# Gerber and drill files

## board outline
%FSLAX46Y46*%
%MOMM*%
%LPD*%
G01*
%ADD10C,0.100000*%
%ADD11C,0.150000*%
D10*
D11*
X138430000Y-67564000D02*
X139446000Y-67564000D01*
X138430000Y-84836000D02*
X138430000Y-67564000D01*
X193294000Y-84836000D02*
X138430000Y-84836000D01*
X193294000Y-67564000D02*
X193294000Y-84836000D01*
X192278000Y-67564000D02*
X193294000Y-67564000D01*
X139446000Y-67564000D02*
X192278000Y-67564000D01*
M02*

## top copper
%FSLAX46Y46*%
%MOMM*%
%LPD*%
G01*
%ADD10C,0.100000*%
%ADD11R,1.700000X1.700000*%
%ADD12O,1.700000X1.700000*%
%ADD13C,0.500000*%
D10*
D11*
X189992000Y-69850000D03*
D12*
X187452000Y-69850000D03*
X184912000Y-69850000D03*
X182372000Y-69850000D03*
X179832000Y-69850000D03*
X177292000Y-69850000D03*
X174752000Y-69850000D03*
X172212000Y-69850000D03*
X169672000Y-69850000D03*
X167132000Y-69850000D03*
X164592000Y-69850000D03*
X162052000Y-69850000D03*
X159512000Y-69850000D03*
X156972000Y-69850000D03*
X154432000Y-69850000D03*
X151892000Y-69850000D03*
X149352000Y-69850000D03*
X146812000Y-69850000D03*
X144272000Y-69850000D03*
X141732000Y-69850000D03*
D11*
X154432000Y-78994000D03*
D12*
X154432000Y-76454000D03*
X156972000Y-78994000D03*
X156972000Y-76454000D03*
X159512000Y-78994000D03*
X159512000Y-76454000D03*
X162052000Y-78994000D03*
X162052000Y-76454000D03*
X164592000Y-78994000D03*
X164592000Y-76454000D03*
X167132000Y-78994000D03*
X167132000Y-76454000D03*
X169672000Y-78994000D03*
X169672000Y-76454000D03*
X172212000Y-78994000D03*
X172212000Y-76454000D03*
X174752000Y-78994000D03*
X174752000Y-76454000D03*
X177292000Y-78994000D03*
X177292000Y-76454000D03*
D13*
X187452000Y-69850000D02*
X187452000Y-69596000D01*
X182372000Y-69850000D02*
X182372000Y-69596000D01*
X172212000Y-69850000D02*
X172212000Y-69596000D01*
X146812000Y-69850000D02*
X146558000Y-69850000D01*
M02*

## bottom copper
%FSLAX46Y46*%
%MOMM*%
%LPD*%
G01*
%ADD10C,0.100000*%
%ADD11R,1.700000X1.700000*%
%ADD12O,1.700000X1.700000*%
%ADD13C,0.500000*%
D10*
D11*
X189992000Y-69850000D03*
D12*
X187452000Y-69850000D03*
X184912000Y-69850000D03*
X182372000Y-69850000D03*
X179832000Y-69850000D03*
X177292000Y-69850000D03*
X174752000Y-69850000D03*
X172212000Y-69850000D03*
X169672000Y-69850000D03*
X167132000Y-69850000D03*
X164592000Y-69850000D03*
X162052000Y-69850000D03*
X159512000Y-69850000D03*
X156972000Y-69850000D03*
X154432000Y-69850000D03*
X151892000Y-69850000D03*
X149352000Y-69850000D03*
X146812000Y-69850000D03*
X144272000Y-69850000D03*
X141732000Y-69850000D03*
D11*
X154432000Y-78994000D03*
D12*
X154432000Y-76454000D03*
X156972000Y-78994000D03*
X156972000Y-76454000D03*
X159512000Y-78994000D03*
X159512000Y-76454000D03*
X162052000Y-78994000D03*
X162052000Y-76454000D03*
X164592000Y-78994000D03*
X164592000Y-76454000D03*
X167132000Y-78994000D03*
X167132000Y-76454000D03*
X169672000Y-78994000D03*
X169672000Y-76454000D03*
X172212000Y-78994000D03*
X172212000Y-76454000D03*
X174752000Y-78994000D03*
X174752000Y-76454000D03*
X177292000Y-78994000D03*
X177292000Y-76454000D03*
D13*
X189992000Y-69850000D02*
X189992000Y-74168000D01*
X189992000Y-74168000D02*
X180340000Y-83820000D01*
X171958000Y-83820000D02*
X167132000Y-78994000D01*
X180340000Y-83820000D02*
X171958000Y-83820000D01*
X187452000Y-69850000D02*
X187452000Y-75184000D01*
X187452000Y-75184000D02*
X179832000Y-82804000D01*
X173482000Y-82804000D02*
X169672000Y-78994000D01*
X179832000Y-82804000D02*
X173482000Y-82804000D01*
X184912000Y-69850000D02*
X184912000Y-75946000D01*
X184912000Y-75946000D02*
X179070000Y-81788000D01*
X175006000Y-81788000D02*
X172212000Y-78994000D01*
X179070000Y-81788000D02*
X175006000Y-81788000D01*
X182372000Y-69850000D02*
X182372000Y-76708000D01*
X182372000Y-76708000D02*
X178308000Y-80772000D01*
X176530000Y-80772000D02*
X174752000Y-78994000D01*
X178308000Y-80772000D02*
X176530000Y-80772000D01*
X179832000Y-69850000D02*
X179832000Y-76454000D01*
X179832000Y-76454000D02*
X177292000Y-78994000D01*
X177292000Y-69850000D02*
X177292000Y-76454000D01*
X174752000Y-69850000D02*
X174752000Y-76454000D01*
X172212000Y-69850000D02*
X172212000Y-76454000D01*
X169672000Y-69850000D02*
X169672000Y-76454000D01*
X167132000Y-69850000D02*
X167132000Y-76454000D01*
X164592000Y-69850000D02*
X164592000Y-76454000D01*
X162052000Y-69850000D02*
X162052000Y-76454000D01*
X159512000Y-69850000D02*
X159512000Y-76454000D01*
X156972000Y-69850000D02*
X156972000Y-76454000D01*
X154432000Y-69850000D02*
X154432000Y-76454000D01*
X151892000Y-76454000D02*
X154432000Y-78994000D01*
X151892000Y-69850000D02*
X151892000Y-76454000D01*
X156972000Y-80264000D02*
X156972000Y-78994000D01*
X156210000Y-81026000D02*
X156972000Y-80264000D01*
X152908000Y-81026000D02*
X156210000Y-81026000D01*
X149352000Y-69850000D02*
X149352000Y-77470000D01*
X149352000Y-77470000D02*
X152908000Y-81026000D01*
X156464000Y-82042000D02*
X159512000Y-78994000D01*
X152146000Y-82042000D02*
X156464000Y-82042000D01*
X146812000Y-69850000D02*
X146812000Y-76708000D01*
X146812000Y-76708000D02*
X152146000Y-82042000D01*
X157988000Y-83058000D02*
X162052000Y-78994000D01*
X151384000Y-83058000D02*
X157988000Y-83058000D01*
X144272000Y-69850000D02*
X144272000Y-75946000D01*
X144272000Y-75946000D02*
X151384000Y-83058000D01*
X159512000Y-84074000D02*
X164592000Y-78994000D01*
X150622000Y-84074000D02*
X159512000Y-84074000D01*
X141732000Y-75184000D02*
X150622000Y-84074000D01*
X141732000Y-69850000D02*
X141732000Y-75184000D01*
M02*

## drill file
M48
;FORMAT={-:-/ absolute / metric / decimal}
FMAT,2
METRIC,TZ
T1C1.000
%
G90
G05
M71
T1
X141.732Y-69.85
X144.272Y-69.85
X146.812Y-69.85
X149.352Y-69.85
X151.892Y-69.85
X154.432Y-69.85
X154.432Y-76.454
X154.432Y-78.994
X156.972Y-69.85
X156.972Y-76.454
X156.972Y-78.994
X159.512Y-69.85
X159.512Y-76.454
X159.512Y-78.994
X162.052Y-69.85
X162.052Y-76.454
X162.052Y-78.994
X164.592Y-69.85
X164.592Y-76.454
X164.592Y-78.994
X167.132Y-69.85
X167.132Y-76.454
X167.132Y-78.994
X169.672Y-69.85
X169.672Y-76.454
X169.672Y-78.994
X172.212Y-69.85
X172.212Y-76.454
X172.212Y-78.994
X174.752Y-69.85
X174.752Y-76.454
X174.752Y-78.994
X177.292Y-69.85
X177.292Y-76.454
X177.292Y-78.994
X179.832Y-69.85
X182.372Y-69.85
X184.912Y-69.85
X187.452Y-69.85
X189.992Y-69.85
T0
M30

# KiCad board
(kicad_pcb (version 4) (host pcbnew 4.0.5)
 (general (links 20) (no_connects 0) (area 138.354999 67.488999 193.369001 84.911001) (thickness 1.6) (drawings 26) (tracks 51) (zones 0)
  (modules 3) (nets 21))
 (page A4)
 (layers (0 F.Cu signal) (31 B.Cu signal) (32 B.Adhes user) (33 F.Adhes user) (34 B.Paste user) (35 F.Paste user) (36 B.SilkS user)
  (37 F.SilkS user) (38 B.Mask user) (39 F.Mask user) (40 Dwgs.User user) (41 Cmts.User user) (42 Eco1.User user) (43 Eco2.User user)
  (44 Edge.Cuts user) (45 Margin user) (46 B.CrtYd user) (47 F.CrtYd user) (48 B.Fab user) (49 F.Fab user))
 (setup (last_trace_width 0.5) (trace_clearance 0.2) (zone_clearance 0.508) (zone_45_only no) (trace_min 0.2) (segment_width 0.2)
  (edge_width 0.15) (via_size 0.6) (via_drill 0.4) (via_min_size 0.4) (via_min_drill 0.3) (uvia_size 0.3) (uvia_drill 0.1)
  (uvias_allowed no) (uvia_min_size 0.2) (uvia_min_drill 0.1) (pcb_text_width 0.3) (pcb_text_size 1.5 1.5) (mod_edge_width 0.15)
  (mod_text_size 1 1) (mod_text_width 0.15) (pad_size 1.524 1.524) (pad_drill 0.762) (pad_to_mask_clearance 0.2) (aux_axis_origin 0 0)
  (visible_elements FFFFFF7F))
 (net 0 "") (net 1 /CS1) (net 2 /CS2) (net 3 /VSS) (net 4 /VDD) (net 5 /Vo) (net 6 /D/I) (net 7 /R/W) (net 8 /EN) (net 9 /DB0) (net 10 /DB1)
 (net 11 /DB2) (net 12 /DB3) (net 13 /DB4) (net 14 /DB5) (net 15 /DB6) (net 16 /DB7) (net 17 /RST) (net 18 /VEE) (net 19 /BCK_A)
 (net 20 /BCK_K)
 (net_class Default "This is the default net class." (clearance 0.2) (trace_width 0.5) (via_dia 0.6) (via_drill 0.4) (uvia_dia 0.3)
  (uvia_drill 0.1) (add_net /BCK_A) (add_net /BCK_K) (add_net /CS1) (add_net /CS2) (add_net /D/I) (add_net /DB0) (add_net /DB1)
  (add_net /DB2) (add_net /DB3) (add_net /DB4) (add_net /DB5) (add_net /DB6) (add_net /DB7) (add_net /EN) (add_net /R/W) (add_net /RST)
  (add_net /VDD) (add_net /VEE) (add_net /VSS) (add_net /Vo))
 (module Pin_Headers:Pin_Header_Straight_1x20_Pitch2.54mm (layer F.Cu) (at 189.992 69.85 270)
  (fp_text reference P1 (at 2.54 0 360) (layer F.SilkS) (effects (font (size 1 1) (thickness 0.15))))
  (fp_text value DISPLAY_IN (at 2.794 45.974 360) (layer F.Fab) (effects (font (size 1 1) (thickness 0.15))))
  (pad 1 thru_hole rect (at 0 0 270) (size 1.7 1.7) (drill 1) (layers *.Cu *.Mask) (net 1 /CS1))
  (pad 2 thru_hole oval (at 0 2.54 270) (size 1.7 1.7) (drill 1) (layers *.Cu *.Mask) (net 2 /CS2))
  (pad 3 thru_hole oval (at 0 5.08 270) (size 1.7 1.7) (drill 1) (layers *.Cu *.Mask) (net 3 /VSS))
  (pad 4 thru_hole oval (at 0 7.62 270) (size 1.7 1.7) (drill 1) (layers *.Cu *.Mask) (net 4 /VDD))
  (pad 5 thru_hole oval (at 0 10.16 270) (size 1.7 1.7) (drill 1) (layers *.Cu *.Mask) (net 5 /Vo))
  (pad 6 thru_hole oval (at 0 12.7 270) (size 1.7 1.7) (drill 1) (layers *.Cu *.Mask) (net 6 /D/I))
  (pad 7 thru_hole oval (at 0 15.24 270) (size 1.7 1.7) (drill 1) (layers *.Cu *.Mask) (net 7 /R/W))
  (pad 8 thru_hole oval (at 0 17.78 270) (size 1.7 1.7) (drill 1) (layers *.Cu *.Mask) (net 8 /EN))
  (pad 9 thru_hole oval (at 0 20.32 270) (size 1.7 1.7) (drill 1) (layers *.Cu *.Mask) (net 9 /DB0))
  (pad 10 thru_hole oval (at 0 22.86 270) (size 1.7 1.7) (drill 1) (layers *.Cu *.Mask) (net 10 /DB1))
  (pad 11 thru_hole oval (at 0 25.4 270) (size 1.7 1.7) (drill 1) (layers *.Cu *.Mask) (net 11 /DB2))
  (pad 12 thru_hole oval (at 0 27.94 270) (size 1.7 1.7) (drill 1) (layers *.Cu *.Mask) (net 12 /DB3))
  (pad 13 thru_hole oval (at 0 30.48 270) (size 1.7 1.7) (drill 1) (layers *.Cu *.Mask) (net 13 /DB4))
  (pad 14 thru_hole oval (at 0 33.02 270) (size 1.7 1.7) (drill 1) (layers *.Cu *.Mask) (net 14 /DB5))
  (pad 15 thru_hole oval (at 0 35.56 270) (size 1.7 1.7) (drill 1) (layers *.Cu *.Mask) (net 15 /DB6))
  (pad 16 thru_hole oval (at 0 38.1 270) (size 1.7 1.7) (drill 1) (layers *.Cu *.Mask) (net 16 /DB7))
  (pad 17 thru_hole oval (at 0 40.64 270) (size 1.7 1.7) (drill 1) (layers *.Cu *.Mask) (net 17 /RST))
  (pad 18 thru_hole oval (at 0 43.18 270) (size 1.7 1.7) (drill 1) (layers *.Cu *.Mask) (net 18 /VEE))
  (pad 19 thru_hole oval (at 0 45.72 270) (size 1.7 1.7) (drill 1) (layers *.Cu *.Mask) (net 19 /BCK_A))
  (pad 20 thru_hole oval (at 0 48.26 270) (size 1.7 1.7) (drill 1) (layers *.Cu *.Mask) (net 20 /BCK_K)))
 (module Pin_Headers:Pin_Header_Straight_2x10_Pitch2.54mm (layer F.Cu) (at 154.432 78.994 90)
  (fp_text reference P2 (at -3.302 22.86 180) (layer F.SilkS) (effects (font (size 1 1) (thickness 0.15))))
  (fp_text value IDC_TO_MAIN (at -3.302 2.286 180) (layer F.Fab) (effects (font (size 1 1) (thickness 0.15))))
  (pad 1 thru_hole rect (at 0 0 90) (size 1.7 1.7) (drill 1) (layers *.Cu *.Mask) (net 16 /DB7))
  (pad 2 thru_hole oval (at 2.54 0 90) (size 1.7 1.7) (drill 1) (layers *.Cu *.Mask) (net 15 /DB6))
  (pad 3 thru_hole oval (at 0 2.54 90) (size 1.7 1.7) (drill 1) (layers *.Cu *.Mask) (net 17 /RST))
  (pad 4 thru_hole oval (at 2.54 2.54 90) (size 1.7 1.7) (drill 1) (layers *.Cu *.Mask) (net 14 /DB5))
  (pad 5 thru_hole oval (at 0 5.08 90) (size 1.7 1.7) (drill 1) (layers *.Cu *.Mask) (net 18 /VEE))
  (pad 6 thru_hole oval (at 2.54 5.08 90) (size 1.7 1.7) (drill 1) (layers *.Cu *.Mask) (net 13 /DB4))
  (pad 7 thru_hole oval (at 0 7.62 90) (size 1.7 1.7) (drill 1) (layers *.Cu *.Mask) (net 19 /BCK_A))
  (pad 8 thru_hole oval (at 2.54 7.62 90) (size 1.7 1.7) (drill 1) (layers *.Cu *.Mask) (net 12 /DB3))
  (pad 9 thru_hole oval (at 0 10.16 90) (size 1.7 1.7) (drill 1) (layers *.Cu *.Mask) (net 20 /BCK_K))
  (pad 10 thru_hole oval (at 2.54 10.16 90) (size 1.7 1.7) (drill 1) (layers *.Cu *.Mask) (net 11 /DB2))
  (pad 11 thru_hole oval (at 0 12.7 90) (size 1.7 1.7) (drill 1) (layers *.Cu *.Mask) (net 1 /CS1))
  (pad 12 thru_hole oval (at 2.54 12.7 90) (size 1.7 1.7) (drill 1) (layers *.Cu *.Mask) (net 10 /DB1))
  (pad 13 thru_hole oval (at 0 15.24 90) (size 1.7 1.7) (drill 1) (layers *.Cu *.Mask) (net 2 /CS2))
  (pad 14 thru_hole oval (at 2.54 15.24 90) (size 1.7 1.7) (drill 1) (layers *.Cu *.Mask) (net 9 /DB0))
  (pad 15 thru_hole oval (at 0 17.78 90) (size 1.7 1.7) (drill 1) (layers *.Cu *.Mask) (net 3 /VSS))
  (pad 16 thru_hole oval (at 2.54 17.78 90) (size 1.7 1.7) (drill 1) (layers *.Cu *.Mask) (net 8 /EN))
  (pad 17 thru_hole oval (at 0 20.32 90) (size 1.7 1.7) (drill 1) (layers *.Cu *.Mask) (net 4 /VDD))
  (pad 18 thru_hole oval (at 2.54 20.32 90) (size 1.7 1.7) (drill 1) (layers *.Cu *.Mask) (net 7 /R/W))
  (pad 19 thru_hole oval (at 0 22.86 90) (size 1.7 1.7) (drill 1) (layers *.Cu *.Mask) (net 5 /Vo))
  (pad 20 thru_hole oval (at 2.54 22.86 90) (size 1.7 1.7) (drill 1) (layers *.Cu *.Mask) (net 6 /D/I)))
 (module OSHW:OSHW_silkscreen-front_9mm (layer F.Cu) (at 145.288 78.994)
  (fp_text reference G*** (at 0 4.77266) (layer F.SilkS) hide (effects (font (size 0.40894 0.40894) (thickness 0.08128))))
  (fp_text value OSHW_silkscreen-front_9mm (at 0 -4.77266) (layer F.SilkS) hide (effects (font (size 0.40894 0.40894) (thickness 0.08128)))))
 (gr_line (start 138.43 67.564) (end 139.446 67.564) (angle 90) (layer Edge.Cuts) (width 0.15))
 (gr_line (start 138.43 84.836) (end 138.43 67.564) (angle 90) (layer Edge.Cuts) (width 0.15))
 (gr_line (start 193.294 84.836) (end 138.43 84.836) (angle 90) (layer Edge.Cuts) (width 0.15))
 (gr_line (start 193.294 67.564) (end 193.294 84.836) (angle 90) (layer Edge.Cuts) (width 0.15))
 (gr_line (start 192.278 67.564) (end 193.294 67.564) (angle 90) (layer Edge.Cuts) (width 0.15))
 (gr_line (start 139.446 67.564) (end 192.278 67.564) (angle 90) (layer Edge.Cuts) (width 0.15))
 (segment (start 189.992 69.85) (end 189.992 74.168) (width 0.5) (layer B.Cu) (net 1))
 (segment (start 189.992 74.168) (end 180.34 83.82) (width 0.5) (layer B.Cu) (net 1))
 (segment (start 171.958 83.82) (end 167.132 78.994) (width 0.5) (layer B.Cu) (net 1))
 (segment (start 180.34 83.82) (end 171.958 83.82) (width 0.5) (layer B.Cu) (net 1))
 (segment (start 187.452 69.85) (end 187.452 69.596) (width 0.5) (layer F.Cu) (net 2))
 (segment (start 187.452 69.85) (end 187.452 75.184) (width 0.5) (layer B.Cu) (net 2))
 (segment (start 187.452 75.184) (end 179.832 82.804) (width 0.5) (layer B.Cu) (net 2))
 (segment (start 173.482 82.804) (end 169.672 78.994) (width 0.5) (layer B.Cu) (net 2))
 (segment (start 179.832 82.804) (end 173.482 82.804) (width 0.5) (layer B.Cu) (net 2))
 (segment (start 184.912 69.85) (end 184.912 75.946) (width 0.5) (layer B.Cu) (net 3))
 (segment (start 184.912 75.946) (end 179.07 81.788) (width 0.5) (layer B.Cu) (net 3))
 (segment (start 175.006 81.788) (end 172.212 78.994) (width 0.5) (layer B.Cu) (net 3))
 (segment (start 179.07 81.788) (end 175.006 81.788) (width 0.5) (layer B.Cu) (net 3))
 (segment (start 182.372 69.85) (end 182.372 69.596) (width 0.5) (layer F.Cu) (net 4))
 (segment (start 182.372 69.85) (end 182.372 76.708) (width 0.5) (layer B.Cu) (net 4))
 (segment (start 182.372 76.708) (end 178.308 80.772) (width 0.5) (layer B.Cu) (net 4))
 (segment (start 176.53 80.772) (end 174.752 78.994) (width 0.5) (layer B.Cu) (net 4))
 (segment (start 178.308 80.772) (end 176.53 80.772) (width 0.5) (layer B.Cu) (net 4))
 (segment (start 179.832 69.85) (end 179.832 76.454) (width 0.5) (layer B.Cu) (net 5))
 (segment (start 179.832 76.454) (end 177.292 78.994) (width 0.5) (layer B.Cu) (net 5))
 (segment (start 177.292 69.85) (end 177.292 76.454) (width 0.5) (layer B.Cu) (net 6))
 (segment (start 174.752 69.85) (end 174.752 76.454) (width 0.5) (layer B.Cu) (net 7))
 (segment (start 172.212 69.85) (end 172.212 69.596) (width 0.5) (layer F.Cu) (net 8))
 (segment (start 172.212 69.85) (end 172.212 76.454) (width 0.5) (layer B.Cu) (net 8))
 (segment (start 169.672 69.85) (end 169.672 76.454) (width 0.5) (layer B.Cu) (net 9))
 (segment (start 167.132 69.85) (end 167.132 76.454) (width 0.5) (layer B.Cu) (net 10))
 (segment (start 164.592 69.85) (end 164.592 76.454) (width 0.5) (layer B.Cu) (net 11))
 (segment (start 162.052 69.85) (end 162.052 76.454) (width 0.5) (layer B.Cu) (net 12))
 (segment (start 159.512 69.85) (end 159.512 76.454) (width 0.5) (layer B.Cu) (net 13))
 (segment (start 156.972 69.85) (end 156.972 76.454) (width 0.5) (layer B.Cu) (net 14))
 (segment (start 154.432 69.85) (end 154.432 76.454) (width 0.5) (layer B.Cu) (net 15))
 (segment (start 151.892 76.454) (end 154.432 78.994) (width 0.5) (layer B.Cu) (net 16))
 (segment (start 151.892 69.85) (end 151.892 76.454) (width 0.5) (layer B.Cu) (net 16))
 (segment (start 156.972 80.264) (end 156.972 78.994) (width 0.5) (layer B.Cu) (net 17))
 (segment (start 156.21 81.026) (end 156.972 80.264) (width 0.5) (layer B.Cu) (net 17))
 (segment (start 152.908 81.026) (end 156.21 81.026) (width 0.5) (layer B.Cu) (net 17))
 (segment (start 149.352 69.85) (end 149.352 77.47) (width 0.5) (layer B.Cu) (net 17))
 (segment (start 149.352 77.47) (end 152.908 81.026) (width 0.5) (layer B.Cu) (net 17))
 (segment (start 146.812 69.85) (end 146.558 69.85) (width 0.5) (layer F.Cu) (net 18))
 (segment (start 156.464 82.042) (end 159.512 78.994) (width 0.5) (layer B.Cu) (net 18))
 (segment (start 152.146 82.042) (end 156.464 82.042) (width 0.5) (layer B.Cu) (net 18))
 (segment (start 146.812 69.85) (end 146.812 76.708) (width 0.5) (layer B.Cu) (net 18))
 (segment (start 146.812 76.708) (end 152.146 82.042) (width 0.5) (layer B.Cu) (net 18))
 (segment (start 157.988 83.058) (end 162.052 78.994) (width 0.5) (layer B.Cu) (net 19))
 (segment (start 151.384 83.058) (end 157.988 83.058) (width 0.5) (layer B.Cu) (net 19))
 (segment (start 144.272 69.85) (end 144.272 75.946) (width 0.5) (layer B.Cu) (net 19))
 (segment (start 144.272 75.946) (end 151.384 83.058) (width 0.5) (layer B.Cu) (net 19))
 (segment (start 159.512 84.074) (end 164.592 78.994) (width 0.5) (layer B.Cu) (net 20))
 (segment (start 150.622 84.074) (end 159.512 84.074) (width 0.5) (layer B.Cu) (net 20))
 (segment (start 141.732 75.184) (end 150.622 84.074) (width 0.5) (layer B.Cu) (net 20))
 (segment (start 141.732 69.85) (end 141.732 75.184) (width 0.5) (layer B.Cu) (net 20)))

